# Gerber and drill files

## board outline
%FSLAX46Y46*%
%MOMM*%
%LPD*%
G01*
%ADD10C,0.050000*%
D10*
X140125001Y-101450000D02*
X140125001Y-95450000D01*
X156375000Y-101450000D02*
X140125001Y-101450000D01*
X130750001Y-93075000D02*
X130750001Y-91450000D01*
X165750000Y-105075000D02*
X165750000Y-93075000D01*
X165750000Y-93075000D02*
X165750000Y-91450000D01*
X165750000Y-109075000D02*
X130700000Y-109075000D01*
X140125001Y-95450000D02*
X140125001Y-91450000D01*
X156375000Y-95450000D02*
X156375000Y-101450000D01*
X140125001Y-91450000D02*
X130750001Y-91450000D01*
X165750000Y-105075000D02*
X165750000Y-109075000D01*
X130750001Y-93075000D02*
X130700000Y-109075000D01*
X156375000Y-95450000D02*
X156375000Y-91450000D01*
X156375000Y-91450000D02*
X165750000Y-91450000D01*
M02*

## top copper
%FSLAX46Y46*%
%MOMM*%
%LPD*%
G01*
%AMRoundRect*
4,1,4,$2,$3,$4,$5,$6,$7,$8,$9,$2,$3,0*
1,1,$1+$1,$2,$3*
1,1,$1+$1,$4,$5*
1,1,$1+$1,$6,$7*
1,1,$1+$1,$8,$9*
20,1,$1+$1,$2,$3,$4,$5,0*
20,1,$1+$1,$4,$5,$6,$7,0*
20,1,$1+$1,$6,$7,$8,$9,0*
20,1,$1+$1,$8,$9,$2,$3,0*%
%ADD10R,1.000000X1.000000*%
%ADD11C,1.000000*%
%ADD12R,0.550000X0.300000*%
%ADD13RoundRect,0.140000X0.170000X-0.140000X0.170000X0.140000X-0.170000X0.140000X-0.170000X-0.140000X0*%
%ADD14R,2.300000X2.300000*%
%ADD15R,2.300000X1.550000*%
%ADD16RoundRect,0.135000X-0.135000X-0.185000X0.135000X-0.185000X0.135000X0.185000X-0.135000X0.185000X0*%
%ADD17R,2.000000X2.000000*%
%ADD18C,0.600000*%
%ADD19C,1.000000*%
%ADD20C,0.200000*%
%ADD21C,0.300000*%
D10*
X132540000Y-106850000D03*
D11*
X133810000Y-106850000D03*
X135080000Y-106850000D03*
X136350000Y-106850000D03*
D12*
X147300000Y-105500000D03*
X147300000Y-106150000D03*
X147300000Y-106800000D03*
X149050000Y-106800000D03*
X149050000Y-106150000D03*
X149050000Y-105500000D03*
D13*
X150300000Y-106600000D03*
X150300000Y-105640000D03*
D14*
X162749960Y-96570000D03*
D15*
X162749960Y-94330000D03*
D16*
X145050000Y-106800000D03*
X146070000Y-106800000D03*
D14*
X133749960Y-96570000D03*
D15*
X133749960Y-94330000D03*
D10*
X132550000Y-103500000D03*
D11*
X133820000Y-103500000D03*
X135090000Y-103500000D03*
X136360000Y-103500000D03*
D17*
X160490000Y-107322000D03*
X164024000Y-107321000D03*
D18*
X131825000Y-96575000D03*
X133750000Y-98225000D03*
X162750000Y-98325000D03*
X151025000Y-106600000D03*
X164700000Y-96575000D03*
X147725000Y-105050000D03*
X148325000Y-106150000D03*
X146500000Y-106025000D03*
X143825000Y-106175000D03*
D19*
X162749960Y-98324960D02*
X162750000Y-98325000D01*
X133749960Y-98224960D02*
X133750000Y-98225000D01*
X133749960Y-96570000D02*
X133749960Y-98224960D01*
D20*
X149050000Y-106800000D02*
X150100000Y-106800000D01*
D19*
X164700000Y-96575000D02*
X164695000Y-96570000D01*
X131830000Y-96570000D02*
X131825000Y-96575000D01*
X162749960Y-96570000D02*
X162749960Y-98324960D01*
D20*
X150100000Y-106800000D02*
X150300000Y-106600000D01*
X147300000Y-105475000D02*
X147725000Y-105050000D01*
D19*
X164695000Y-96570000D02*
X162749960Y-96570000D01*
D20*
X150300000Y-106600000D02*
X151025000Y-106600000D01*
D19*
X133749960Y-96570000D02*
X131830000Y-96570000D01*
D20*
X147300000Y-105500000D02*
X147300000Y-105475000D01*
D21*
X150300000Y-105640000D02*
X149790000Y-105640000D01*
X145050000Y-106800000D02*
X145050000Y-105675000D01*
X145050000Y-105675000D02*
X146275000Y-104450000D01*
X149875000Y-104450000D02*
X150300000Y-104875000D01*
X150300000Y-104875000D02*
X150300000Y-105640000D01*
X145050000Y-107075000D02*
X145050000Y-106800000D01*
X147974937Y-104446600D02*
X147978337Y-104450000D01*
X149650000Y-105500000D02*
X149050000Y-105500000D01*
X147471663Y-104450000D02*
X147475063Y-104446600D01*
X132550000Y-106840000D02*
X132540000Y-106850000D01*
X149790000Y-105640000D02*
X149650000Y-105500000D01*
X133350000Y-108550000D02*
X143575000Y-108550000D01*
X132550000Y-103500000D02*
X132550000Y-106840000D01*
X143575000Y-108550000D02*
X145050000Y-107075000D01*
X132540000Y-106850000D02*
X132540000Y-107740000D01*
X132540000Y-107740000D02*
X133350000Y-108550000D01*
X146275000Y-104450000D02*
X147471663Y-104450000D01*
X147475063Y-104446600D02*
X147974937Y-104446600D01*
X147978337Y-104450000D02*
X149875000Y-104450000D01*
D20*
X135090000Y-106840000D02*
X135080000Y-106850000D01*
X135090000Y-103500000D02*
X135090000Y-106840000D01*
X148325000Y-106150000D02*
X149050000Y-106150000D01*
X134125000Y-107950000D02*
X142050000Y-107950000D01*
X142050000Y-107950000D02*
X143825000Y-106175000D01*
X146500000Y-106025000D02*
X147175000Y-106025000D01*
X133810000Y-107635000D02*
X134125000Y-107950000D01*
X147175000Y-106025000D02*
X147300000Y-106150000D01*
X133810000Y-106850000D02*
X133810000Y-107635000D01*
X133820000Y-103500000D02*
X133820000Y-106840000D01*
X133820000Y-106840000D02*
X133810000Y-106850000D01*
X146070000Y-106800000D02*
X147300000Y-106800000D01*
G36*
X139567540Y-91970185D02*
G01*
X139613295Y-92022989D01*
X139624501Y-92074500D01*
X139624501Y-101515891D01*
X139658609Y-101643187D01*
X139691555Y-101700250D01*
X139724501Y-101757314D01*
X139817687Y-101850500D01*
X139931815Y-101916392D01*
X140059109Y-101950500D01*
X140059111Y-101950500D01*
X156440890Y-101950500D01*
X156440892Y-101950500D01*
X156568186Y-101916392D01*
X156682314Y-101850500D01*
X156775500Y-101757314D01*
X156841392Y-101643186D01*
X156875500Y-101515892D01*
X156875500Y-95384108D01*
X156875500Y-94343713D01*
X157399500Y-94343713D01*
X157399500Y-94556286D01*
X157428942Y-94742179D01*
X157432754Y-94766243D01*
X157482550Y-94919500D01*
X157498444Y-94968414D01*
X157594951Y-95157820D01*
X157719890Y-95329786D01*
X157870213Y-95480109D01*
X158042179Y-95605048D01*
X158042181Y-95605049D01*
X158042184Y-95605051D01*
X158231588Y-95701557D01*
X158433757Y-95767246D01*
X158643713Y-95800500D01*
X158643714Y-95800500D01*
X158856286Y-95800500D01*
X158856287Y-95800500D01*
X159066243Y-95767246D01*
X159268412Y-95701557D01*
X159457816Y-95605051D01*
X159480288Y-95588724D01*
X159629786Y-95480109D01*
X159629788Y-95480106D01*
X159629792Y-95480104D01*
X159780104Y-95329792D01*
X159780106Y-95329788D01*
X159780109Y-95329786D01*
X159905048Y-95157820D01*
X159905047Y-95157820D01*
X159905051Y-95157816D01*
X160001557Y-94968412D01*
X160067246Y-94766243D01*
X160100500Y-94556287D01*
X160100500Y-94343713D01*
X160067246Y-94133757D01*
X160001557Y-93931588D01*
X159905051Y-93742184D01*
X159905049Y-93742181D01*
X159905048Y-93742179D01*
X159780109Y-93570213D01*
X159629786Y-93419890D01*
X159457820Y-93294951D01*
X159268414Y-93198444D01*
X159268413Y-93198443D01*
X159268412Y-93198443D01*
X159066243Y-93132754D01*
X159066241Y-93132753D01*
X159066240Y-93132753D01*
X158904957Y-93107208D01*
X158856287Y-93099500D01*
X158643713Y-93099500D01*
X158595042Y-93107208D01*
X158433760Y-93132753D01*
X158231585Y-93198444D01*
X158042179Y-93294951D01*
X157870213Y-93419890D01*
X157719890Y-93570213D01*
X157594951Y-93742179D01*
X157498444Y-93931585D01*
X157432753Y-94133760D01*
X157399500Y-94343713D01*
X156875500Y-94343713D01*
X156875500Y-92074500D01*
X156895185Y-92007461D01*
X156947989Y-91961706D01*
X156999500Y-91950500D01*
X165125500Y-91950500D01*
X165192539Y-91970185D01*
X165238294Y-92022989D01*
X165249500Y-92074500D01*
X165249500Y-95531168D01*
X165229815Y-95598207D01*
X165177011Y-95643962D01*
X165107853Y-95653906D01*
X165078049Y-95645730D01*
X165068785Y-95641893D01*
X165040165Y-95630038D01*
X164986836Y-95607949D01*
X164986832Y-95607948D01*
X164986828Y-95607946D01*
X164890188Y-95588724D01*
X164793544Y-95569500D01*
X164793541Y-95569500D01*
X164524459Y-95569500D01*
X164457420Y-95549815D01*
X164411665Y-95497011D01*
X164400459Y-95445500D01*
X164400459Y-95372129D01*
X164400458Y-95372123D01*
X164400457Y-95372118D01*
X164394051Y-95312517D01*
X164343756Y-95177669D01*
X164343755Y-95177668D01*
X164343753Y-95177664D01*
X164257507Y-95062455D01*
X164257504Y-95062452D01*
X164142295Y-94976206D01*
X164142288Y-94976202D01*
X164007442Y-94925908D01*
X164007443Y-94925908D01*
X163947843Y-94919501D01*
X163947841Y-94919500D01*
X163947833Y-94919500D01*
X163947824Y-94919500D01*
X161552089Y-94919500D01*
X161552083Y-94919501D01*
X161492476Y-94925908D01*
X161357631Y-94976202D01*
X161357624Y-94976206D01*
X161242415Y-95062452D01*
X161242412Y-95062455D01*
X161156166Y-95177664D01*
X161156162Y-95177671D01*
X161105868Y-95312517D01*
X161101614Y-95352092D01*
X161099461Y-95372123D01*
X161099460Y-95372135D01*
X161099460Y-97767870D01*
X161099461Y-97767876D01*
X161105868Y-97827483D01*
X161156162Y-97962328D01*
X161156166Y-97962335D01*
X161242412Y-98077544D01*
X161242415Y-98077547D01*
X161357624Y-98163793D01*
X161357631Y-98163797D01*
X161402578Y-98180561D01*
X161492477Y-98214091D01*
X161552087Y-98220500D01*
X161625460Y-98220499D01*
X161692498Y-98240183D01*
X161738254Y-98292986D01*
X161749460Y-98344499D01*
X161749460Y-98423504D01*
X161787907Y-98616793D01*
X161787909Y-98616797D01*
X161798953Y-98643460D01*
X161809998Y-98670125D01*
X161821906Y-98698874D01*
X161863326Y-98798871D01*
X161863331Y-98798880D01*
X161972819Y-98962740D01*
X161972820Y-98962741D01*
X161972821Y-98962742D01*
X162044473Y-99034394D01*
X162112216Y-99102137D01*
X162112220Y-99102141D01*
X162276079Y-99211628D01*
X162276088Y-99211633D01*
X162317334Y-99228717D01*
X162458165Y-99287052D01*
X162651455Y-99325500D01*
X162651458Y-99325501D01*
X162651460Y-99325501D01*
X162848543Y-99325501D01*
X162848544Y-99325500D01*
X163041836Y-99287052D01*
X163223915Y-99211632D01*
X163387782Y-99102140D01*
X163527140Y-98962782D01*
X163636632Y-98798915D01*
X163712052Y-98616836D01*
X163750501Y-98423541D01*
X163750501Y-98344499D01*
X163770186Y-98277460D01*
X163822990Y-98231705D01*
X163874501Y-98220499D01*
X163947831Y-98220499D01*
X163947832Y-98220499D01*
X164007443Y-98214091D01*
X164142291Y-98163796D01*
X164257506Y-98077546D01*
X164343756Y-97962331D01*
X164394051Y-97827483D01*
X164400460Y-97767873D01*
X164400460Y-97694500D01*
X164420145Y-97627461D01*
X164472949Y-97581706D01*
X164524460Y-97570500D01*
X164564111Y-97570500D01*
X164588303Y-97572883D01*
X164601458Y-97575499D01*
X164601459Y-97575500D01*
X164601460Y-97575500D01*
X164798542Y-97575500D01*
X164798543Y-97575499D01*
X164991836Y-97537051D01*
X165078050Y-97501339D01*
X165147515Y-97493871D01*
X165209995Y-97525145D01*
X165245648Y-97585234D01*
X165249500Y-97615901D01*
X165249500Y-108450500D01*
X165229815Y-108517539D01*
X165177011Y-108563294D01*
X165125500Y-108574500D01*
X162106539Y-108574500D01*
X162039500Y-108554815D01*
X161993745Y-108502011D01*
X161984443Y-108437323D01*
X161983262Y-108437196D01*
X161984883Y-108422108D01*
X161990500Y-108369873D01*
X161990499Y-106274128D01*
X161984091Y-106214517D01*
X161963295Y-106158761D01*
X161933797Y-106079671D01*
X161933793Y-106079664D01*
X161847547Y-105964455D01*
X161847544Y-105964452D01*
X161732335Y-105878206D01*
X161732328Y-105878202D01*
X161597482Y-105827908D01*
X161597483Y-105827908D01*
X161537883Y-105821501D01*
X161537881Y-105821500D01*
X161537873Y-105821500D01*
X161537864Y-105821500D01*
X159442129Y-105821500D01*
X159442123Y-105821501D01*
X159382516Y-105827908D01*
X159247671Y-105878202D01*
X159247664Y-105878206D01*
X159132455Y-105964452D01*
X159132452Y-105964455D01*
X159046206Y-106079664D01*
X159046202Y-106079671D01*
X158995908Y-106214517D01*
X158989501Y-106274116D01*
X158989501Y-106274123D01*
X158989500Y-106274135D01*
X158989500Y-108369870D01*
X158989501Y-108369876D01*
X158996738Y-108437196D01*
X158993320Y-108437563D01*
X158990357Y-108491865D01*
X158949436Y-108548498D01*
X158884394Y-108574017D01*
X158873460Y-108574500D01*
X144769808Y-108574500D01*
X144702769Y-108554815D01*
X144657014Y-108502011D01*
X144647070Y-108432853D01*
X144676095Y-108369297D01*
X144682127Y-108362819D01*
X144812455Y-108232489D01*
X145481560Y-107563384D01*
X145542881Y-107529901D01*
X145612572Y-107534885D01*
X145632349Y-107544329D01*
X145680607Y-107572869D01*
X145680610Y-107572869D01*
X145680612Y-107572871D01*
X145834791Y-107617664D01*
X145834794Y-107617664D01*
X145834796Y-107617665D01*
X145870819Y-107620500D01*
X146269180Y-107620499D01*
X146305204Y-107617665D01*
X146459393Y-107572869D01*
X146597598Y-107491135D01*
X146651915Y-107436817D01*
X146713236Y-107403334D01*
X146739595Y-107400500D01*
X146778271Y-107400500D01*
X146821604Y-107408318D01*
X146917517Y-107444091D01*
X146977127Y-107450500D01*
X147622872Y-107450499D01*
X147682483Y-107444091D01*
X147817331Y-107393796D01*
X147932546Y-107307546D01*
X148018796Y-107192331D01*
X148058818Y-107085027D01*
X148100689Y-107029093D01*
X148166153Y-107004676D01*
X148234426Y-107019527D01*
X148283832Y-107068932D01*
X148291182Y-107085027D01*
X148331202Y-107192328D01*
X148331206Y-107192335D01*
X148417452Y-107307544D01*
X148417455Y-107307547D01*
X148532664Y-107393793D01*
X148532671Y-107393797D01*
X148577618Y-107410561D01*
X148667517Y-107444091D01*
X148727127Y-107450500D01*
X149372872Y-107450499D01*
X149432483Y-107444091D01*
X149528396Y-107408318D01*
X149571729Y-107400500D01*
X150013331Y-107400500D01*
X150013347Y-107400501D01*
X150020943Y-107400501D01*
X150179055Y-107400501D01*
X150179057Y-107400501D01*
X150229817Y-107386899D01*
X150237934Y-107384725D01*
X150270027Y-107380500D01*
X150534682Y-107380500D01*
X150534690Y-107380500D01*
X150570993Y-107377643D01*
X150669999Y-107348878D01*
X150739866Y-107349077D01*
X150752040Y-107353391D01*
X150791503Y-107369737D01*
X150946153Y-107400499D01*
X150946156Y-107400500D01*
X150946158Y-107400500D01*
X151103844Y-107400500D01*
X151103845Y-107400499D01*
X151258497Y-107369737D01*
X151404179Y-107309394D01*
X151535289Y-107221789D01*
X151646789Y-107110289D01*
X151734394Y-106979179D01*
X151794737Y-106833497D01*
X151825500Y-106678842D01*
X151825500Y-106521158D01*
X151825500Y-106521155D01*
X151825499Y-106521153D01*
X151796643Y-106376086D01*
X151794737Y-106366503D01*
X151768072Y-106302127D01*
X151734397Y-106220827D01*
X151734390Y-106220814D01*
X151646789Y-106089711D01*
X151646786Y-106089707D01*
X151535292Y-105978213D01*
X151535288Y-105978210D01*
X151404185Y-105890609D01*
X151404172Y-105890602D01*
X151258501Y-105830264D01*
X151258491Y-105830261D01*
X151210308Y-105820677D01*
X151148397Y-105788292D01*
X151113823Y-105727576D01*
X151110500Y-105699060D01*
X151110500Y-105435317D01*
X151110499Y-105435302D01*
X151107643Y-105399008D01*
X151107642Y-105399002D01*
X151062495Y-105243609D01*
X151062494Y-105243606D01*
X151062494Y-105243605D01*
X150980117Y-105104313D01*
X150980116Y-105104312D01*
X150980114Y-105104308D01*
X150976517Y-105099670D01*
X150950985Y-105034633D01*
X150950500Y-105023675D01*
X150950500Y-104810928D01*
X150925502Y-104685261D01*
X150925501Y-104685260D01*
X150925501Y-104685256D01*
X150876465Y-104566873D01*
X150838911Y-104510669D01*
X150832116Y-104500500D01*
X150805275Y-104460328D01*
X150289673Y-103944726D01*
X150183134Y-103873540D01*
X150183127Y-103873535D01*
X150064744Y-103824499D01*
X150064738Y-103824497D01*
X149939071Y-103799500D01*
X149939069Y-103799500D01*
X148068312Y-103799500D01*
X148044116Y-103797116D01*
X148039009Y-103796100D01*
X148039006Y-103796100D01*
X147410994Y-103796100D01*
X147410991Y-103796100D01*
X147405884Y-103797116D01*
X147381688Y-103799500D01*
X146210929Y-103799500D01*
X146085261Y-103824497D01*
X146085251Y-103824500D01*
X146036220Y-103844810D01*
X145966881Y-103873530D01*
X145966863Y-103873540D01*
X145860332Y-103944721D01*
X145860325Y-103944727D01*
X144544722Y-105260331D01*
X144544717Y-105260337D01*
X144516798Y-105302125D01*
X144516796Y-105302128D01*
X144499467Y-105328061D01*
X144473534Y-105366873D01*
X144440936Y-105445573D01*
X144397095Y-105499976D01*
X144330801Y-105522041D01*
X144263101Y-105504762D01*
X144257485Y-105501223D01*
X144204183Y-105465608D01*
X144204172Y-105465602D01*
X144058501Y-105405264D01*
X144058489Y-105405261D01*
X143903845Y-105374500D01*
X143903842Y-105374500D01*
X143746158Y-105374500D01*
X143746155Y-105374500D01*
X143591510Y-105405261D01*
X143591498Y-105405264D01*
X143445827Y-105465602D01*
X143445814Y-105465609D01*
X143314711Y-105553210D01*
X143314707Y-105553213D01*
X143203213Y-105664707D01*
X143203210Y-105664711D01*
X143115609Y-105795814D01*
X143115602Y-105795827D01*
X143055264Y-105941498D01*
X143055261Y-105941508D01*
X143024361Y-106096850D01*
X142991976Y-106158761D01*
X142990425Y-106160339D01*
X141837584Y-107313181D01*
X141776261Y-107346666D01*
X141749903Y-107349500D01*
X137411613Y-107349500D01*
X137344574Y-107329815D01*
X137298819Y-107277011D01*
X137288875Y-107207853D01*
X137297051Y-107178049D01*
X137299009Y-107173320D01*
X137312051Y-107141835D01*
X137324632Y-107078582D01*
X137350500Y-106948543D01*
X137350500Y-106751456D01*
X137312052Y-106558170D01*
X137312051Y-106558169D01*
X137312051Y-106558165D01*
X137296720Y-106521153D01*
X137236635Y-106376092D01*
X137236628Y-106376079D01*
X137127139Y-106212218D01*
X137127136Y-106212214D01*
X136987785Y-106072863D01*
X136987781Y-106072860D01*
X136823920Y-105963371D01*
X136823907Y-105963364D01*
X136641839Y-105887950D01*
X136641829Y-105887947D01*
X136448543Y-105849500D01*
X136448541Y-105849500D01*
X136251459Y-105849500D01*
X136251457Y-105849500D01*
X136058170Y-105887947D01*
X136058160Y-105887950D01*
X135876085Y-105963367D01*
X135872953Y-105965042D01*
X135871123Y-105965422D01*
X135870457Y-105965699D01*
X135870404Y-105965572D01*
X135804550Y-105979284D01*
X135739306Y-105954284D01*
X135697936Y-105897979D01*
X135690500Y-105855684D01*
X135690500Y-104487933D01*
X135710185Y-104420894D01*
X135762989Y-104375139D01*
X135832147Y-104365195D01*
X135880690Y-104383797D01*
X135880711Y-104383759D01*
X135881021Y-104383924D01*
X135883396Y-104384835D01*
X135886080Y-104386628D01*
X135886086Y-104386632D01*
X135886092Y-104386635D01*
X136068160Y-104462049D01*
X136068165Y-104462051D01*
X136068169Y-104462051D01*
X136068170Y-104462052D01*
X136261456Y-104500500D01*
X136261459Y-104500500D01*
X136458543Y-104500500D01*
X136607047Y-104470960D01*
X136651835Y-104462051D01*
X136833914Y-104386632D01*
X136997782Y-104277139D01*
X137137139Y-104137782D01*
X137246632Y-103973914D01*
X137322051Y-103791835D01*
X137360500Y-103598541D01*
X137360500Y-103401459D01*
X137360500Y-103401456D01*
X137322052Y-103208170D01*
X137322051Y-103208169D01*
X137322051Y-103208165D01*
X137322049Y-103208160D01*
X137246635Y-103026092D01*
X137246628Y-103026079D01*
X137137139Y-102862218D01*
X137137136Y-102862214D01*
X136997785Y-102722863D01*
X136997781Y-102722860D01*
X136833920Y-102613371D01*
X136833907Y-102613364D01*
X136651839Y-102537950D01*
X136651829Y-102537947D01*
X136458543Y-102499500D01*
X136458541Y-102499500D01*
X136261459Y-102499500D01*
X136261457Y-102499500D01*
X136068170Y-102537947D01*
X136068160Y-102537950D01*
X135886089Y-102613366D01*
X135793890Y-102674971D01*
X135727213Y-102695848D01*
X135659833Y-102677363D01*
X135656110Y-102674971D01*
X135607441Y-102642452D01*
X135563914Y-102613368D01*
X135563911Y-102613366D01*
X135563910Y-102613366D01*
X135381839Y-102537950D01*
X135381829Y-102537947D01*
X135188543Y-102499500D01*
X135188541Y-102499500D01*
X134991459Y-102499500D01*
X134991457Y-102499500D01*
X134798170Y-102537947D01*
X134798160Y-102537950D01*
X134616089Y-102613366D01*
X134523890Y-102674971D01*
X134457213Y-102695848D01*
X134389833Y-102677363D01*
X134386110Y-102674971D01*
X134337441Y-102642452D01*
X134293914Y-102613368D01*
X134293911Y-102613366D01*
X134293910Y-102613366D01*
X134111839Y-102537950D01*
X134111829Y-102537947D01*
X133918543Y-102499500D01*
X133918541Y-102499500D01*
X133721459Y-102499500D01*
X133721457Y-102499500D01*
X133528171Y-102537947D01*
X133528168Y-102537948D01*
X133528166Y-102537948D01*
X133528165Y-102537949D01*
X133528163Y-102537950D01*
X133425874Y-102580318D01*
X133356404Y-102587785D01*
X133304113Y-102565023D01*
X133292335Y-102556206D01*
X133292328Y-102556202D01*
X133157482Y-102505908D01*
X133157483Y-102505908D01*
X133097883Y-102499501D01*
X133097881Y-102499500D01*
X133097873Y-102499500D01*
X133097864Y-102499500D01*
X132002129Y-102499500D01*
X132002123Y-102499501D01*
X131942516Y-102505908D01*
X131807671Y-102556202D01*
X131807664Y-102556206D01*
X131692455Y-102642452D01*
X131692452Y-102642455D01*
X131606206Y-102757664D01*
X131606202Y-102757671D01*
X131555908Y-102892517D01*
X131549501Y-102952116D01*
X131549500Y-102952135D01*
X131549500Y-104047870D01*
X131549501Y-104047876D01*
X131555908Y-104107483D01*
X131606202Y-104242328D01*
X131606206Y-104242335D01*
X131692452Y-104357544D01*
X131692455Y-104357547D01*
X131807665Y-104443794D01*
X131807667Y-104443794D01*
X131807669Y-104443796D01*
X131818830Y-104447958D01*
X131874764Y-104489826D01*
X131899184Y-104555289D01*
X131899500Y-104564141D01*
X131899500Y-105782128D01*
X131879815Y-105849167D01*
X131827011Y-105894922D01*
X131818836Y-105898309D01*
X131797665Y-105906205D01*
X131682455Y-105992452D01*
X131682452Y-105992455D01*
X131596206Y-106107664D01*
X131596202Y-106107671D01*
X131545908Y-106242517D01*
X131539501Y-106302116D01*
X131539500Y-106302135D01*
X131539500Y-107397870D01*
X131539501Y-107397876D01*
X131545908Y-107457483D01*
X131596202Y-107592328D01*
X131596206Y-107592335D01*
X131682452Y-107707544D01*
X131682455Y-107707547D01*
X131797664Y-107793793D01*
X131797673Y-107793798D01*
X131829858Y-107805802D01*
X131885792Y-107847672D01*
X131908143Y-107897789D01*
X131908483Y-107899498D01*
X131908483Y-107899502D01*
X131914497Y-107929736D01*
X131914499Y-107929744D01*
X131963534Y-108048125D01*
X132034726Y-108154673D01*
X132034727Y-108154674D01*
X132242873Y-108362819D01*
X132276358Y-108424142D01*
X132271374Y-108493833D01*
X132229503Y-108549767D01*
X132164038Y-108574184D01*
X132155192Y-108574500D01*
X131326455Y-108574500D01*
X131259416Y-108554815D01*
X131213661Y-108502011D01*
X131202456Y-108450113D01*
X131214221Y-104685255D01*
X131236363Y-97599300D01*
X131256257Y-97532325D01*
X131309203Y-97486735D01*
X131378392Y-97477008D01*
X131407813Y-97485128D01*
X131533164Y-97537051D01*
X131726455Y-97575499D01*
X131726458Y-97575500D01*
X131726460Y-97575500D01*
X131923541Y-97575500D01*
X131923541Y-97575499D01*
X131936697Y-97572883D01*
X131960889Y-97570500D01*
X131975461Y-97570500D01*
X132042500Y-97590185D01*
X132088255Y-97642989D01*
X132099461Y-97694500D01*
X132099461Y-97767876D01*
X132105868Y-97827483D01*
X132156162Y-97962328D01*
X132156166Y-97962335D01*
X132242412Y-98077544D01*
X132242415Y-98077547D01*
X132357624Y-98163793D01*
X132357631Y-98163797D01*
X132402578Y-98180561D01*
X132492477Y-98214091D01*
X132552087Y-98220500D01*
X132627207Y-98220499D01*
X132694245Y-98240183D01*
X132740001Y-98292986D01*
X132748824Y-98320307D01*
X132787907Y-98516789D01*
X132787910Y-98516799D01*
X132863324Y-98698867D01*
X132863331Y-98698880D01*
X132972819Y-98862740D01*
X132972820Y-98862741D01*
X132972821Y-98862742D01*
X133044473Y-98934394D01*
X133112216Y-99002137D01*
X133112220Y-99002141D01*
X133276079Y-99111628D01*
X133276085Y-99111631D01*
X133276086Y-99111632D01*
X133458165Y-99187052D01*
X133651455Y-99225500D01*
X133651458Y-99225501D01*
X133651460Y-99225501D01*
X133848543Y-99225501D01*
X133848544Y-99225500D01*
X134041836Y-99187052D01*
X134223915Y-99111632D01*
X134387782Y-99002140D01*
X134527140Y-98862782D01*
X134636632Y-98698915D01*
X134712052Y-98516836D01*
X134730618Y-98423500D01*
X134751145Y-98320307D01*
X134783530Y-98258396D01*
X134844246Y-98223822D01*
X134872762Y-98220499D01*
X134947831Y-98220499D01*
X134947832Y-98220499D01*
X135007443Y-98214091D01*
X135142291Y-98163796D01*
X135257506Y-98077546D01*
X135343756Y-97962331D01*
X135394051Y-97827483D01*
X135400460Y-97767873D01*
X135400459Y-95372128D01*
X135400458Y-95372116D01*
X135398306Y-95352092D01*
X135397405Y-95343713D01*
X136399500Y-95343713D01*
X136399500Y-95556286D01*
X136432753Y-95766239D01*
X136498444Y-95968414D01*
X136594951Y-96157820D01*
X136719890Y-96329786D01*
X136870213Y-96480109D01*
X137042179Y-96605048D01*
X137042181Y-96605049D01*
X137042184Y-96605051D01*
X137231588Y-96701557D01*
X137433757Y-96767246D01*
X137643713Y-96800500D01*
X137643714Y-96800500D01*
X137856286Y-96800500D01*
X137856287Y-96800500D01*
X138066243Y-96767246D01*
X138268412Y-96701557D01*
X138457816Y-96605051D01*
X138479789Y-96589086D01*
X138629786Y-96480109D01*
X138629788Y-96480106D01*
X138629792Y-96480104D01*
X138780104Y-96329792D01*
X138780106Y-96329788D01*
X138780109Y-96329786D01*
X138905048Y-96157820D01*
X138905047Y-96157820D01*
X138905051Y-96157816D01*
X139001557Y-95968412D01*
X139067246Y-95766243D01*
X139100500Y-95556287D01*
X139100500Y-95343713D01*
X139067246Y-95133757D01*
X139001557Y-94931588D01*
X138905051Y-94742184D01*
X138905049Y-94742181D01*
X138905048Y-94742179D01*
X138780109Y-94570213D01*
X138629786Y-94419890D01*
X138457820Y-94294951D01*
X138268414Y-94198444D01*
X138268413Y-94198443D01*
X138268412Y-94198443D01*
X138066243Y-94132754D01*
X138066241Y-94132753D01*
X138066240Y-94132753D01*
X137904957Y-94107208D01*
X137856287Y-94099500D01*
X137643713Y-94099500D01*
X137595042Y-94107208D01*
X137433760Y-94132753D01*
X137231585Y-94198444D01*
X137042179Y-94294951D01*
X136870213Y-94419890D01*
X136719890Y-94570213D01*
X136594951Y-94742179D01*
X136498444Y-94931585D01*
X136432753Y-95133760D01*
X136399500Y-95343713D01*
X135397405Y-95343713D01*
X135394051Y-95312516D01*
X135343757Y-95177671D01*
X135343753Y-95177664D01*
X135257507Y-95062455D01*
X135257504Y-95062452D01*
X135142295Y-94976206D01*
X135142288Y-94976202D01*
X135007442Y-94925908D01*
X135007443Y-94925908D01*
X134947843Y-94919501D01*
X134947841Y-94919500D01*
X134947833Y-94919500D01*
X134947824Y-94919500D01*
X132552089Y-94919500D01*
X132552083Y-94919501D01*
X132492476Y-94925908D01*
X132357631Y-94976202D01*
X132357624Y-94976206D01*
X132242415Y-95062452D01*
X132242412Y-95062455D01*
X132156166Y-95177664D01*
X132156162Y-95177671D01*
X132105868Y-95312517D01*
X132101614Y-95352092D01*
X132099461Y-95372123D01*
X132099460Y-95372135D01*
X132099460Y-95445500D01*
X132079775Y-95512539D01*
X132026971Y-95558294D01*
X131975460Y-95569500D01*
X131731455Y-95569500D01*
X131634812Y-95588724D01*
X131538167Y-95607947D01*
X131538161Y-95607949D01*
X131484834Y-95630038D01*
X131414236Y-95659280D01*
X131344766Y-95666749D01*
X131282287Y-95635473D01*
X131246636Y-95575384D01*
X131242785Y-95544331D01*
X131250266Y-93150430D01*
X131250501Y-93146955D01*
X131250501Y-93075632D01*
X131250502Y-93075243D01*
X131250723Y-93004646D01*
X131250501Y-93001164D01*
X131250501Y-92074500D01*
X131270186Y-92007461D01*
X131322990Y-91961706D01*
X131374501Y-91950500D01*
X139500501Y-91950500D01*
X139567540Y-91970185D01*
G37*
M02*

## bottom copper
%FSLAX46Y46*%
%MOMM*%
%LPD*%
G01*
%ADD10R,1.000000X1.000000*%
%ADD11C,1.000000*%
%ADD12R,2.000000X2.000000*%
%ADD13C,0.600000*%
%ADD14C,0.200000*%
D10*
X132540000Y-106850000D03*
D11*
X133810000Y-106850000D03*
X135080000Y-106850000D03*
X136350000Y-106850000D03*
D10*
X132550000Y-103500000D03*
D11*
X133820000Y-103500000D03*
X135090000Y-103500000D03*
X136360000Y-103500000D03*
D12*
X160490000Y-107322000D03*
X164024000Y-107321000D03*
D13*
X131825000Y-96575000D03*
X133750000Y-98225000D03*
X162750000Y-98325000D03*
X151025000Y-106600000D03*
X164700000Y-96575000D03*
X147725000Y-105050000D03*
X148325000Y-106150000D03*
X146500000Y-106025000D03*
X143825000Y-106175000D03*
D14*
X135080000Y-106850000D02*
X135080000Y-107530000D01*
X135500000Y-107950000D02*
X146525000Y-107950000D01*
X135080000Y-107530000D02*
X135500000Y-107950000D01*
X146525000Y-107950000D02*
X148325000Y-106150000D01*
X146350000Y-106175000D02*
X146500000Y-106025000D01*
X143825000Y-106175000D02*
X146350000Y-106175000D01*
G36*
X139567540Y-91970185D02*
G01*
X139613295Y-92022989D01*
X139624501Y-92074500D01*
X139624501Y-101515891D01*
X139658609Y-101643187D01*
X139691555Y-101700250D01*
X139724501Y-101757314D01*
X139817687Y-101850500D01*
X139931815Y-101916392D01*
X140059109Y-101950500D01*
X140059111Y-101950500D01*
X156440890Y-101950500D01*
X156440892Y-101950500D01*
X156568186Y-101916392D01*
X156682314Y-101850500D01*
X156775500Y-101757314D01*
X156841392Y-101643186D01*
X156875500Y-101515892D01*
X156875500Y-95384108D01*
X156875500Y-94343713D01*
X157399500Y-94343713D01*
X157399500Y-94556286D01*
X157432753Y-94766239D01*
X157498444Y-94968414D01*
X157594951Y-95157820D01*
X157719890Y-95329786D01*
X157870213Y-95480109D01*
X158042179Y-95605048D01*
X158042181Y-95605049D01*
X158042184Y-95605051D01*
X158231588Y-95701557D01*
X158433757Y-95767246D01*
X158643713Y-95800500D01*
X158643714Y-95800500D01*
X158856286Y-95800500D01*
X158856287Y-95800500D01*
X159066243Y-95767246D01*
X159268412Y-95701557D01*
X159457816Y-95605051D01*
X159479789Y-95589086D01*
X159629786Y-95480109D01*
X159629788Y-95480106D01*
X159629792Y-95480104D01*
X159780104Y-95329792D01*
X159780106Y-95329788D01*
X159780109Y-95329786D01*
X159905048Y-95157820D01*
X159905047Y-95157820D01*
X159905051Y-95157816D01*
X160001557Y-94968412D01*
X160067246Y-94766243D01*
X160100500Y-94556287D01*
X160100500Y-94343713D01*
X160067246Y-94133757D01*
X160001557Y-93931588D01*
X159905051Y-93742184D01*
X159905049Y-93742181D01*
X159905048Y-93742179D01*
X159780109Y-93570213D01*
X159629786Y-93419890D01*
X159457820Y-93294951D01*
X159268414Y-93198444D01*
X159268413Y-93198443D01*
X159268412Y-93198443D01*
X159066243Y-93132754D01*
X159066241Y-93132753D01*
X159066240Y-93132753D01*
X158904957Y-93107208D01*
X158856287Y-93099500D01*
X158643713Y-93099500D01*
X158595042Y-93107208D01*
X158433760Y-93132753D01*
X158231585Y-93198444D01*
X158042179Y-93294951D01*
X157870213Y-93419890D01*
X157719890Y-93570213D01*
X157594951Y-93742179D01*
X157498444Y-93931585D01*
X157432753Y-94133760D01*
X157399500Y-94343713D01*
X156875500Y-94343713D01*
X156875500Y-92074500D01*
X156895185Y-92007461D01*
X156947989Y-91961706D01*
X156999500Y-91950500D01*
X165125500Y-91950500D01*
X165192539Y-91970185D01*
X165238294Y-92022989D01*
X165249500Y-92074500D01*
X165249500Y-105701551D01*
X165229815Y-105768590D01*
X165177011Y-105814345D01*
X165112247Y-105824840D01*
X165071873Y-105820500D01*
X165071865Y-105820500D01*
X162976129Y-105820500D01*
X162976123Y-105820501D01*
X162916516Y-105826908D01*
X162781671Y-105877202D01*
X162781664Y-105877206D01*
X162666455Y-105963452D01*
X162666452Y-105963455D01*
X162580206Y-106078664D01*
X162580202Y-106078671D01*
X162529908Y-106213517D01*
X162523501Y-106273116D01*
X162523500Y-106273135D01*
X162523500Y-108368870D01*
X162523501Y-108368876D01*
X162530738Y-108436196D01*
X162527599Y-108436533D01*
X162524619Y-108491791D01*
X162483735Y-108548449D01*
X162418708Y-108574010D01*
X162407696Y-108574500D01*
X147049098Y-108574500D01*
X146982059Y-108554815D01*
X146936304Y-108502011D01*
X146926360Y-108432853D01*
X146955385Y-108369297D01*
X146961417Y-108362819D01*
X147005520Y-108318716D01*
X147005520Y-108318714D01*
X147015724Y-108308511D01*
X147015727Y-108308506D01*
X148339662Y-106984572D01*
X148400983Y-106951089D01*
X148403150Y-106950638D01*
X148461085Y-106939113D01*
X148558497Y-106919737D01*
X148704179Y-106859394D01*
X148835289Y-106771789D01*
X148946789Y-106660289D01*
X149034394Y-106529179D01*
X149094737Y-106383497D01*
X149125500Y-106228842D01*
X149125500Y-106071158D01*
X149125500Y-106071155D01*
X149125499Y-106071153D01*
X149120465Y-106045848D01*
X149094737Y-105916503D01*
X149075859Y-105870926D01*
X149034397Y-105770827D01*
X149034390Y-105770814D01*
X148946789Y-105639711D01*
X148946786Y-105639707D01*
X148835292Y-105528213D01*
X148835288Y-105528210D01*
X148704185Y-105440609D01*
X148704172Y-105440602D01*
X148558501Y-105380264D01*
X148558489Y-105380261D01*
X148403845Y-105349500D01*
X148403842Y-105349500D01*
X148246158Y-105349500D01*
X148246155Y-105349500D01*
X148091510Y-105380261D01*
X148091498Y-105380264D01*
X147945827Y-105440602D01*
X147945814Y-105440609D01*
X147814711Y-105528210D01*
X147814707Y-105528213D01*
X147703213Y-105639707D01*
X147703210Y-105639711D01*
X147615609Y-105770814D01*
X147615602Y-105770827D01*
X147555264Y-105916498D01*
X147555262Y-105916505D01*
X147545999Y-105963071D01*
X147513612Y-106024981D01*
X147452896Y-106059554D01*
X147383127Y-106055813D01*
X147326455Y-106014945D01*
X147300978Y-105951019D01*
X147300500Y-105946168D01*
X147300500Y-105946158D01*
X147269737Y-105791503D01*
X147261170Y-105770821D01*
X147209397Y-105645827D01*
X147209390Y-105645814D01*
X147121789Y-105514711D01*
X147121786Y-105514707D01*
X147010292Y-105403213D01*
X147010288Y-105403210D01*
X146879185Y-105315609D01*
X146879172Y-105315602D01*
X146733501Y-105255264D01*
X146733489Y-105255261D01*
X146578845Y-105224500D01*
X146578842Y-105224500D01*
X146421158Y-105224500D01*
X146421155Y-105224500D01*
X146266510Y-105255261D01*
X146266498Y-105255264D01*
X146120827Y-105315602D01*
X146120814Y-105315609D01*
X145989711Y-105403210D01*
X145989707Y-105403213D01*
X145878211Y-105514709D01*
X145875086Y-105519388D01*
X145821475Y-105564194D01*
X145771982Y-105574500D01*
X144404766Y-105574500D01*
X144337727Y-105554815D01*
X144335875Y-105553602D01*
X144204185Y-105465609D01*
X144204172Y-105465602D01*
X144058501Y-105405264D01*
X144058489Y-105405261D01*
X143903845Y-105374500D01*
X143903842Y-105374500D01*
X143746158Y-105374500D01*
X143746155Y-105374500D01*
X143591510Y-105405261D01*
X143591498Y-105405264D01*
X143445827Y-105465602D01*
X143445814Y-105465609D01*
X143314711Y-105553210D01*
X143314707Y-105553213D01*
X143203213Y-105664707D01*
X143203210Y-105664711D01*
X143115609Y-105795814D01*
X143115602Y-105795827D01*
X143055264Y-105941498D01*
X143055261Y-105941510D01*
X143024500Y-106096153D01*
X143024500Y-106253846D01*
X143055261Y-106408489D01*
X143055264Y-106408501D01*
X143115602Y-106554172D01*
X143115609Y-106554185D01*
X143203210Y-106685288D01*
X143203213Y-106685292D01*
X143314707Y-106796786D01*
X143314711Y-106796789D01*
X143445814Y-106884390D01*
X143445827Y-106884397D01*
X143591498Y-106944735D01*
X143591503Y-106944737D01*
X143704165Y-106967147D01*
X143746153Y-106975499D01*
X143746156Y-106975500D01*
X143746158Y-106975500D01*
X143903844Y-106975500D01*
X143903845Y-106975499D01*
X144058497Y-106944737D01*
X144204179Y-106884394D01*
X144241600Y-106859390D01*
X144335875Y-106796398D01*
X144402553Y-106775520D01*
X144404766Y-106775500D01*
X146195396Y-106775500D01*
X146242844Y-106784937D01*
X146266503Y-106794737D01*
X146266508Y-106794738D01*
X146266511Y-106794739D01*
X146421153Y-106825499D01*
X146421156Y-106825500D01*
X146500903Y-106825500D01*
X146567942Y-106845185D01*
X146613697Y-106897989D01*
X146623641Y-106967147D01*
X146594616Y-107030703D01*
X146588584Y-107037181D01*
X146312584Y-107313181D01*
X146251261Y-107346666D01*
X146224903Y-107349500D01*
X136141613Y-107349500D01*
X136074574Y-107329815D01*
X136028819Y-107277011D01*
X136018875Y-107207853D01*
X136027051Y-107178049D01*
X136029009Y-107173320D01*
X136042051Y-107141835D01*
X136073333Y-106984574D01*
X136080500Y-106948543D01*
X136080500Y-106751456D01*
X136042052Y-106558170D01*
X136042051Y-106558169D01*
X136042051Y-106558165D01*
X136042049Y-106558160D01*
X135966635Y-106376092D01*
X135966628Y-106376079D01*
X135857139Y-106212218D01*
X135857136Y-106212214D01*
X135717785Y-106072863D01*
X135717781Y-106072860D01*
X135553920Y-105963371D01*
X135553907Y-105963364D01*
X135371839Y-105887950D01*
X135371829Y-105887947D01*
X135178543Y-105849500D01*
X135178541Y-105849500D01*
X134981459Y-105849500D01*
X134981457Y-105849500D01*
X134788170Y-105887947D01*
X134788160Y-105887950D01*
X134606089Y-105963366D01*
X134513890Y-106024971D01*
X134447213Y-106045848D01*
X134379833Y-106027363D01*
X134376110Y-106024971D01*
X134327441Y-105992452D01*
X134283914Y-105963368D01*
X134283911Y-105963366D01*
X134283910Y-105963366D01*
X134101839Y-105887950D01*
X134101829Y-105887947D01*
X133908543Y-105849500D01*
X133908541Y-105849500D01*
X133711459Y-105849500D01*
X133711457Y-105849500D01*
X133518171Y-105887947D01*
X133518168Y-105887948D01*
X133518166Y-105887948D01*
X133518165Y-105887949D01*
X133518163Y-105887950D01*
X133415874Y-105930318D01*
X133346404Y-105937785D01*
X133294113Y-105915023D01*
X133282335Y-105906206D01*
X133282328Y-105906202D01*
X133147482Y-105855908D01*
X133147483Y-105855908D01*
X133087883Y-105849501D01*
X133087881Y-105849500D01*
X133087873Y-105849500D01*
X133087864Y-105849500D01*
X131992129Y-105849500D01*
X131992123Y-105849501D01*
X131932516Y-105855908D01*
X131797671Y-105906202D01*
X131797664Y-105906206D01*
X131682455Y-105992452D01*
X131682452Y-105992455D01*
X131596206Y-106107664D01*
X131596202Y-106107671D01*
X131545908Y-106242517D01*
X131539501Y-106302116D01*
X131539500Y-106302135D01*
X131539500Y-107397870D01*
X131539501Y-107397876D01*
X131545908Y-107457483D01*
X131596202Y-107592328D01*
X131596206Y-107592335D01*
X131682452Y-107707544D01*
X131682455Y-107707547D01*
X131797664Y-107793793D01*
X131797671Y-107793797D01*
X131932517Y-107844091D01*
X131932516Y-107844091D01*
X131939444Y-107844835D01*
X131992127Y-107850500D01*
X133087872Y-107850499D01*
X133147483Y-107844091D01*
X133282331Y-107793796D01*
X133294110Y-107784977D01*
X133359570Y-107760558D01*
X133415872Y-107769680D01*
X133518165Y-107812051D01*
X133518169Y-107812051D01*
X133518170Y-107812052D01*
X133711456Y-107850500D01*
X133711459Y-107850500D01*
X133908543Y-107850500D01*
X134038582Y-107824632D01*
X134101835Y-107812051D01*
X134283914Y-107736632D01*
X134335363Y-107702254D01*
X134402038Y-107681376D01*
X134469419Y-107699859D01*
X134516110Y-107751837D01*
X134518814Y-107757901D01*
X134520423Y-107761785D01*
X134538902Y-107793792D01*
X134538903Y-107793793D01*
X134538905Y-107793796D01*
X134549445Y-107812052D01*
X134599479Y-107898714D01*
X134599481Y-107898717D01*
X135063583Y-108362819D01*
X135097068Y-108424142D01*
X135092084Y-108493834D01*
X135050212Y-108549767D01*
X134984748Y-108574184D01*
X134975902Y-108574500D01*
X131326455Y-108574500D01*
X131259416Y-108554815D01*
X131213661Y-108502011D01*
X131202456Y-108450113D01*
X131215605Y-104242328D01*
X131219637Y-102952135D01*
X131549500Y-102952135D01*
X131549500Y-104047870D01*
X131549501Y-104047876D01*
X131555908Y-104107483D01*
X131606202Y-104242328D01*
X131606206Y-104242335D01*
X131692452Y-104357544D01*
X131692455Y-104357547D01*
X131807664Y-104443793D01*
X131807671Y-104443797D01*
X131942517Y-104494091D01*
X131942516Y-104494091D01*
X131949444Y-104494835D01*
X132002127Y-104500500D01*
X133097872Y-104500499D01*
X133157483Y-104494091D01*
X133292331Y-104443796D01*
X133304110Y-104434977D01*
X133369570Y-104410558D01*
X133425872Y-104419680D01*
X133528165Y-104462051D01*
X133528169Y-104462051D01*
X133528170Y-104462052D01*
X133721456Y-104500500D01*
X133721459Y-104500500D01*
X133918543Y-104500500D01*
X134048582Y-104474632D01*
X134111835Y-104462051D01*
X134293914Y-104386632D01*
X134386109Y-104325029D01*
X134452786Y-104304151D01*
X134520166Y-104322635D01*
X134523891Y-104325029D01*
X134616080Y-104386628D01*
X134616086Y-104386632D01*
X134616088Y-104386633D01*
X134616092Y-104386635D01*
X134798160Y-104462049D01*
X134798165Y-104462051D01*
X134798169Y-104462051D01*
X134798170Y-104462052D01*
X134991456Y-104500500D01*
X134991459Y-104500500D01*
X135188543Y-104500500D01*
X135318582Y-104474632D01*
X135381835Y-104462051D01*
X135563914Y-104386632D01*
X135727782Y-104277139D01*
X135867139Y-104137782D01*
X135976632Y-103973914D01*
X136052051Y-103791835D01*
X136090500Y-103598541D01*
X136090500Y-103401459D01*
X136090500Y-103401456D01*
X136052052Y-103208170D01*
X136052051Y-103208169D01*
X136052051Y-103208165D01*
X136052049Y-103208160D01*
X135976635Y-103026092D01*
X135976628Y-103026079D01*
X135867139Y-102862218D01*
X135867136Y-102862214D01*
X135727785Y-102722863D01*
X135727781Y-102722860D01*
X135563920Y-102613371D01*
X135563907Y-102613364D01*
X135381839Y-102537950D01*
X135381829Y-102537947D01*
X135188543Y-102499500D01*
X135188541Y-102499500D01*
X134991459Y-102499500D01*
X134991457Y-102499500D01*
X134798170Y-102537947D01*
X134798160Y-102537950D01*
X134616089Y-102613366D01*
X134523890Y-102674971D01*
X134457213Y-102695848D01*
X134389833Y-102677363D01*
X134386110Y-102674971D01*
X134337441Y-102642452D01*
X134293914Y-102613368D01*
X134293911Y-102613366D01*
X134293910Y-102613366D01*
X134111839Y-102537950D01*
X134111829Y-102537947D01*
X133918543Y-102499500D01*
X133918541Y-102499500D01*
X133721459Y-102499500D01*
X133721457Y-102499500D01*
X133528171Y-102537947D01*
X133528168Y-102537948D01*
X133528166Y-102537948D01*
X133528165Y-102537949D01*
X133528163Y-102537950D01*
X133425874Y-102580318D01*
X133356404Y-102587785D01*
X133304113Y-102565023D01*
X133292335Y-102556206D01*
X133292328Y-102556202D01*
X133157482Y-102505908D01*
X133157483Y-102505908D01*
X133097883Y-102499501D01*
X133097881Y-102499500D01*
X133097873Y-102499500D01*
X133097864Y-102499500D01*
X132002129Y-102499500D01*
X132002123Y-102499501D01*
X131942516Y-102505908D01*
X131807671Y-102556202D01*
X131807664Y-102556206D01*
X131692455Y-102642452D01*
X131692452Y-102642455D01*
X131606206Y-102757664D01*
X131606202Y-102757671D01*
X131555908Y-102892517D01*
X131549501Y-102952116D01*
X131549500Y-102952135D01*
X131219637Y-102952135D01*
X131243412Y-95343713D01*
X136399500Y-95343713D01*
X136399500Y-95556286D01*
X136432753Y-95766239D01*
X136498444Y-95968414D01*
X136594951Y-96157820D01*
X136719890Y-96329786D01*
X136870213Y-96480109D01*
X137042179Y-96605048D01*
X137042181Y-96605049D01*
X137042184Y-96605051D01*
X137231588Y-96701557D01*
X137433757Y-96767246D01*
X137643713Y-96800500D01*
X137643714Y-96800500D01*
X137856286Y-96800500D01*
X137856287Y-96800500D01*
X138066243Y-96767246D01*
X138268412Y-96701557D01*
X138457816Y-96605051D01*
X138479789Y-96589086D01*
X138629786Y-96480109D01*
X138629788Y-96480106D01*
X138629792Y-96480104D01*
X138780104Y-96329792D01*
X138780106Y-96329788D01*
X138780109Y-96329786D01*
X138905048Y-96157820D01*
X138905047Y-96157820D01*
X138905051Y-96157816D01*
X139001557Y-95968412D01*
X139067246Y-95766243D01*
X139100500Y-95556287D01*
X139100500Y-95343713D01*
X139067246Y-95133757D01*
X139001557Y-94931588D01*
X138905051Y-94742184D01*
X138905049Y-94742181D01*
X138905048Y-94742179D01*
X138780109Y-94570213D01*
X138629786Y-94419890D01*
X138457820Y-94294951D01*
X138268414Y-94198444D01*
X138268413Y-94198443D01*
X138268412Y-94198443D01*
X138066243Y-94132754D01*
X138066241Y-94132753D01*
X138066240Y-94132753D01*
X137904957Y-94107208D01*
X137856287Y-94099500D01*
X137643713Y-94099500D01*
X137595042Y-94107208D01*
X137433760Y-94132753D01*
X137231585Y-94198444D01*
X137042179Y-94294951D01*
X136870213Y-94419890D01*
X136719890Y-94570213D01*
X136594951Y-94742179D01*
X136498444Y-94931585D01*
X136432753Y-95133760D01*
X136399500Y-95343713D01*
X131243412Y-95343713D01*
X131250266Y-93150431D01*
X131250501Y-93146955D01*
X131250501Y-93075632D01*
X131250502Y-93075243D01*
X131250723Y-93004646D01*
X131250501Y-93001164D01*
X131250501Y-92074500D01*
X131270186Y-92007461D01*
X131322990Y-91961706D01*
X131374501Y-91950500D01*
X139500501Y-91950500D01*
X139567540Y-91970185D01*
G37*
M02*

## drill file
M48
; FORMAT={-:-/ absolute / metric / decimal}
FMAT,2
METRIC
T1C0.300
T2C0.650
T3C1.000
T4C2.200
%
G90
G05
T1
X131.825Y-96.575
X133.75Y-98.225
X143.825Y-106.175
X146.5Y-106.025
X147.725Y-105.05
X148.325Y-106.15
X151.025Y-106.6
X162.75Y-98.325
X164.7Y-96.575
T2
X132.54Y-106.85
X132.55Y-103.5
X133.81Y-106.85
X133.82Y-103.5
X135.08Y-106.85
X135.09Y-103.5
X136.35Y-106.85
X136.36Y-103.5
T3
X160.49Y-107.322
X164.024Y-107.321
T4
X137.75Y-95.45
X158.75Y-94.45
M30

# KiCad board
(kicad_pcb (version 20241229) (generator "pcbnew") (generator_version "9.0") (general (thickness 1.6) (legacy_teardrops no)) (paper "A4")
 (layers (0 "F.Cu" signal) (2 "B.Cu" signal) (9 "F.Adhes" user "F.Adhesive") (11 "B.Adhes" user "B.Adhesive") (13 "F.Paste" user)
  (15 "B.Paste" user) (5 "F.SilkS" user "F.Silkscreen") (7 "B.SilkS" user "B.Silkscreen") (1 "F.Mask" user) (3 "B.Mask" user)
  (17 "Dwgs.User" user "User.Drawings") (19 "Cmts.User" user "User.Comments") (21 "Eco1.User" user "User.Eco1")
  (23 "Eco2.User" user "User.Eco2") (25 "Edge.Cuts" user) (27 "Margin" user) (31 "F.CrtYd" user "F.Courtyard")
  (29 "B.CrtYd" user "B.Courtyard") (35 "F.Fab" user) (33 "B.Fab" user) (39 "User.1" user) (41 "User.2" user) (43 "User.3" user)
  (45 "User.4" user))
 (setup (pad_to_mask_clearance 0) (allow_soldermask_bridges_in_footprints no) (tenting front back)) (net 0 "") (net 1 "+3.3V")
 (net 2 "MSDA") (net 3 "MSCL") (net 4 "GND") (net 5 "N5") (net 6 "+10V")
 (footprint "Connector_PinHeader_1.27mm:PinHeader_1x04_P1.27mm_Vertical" (layer "F.Cu") (at 132.54 106.85 90)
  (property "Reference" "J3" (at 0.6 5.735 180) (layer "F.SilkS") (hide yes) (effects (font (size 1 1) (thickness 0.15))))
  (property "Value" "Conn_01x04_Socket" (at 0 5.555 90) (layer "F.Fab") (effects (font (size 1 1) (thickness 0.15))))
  (pad "1" thru_hole rect (at 0 0 90) (size 1 1) (drill 0.65) (layers "*.Cu" "*.Mask") (remove_unused_layers no) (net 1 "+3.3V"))
  (pad "2" thru_hole circle (at 0 1.27 90) (size 1 1) (drill 0.65) (layers "*.Cu" "*.Mask") (remove_unused_layers no) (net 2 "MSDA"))
  (pad "3" thru_hole circle (at 0 2.54 90) (size 1 1) (drill 0.65) (layers "*.Cu" "*.Mask") (remove_unused_layers no) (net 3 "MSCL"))
  (pad "4" thru_hole circle (at 0 3.81 90) (size 1 1) (drill 0.65) (layers "*.Cu" "*.Mask") (remove_unused_layers no) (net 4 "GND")))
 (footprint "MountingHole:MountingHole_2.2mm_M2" (layer "F.Cu") (at 137.75 95.45)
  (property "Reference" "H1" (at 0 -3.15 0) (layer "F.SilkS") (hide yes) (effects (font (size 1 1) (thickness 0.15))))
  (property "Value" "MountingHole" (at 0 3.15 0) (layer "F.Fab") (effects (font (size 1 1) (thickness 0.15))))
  (pad "" np_thru_hole circle (at 0 0) (size 2.2 2.2) (drill 2.2) (layers "*.Cu" "*.Mask")))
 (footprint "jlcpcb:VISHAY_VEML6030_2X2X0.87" (layer "F.Cu") (at 148.175 106.15)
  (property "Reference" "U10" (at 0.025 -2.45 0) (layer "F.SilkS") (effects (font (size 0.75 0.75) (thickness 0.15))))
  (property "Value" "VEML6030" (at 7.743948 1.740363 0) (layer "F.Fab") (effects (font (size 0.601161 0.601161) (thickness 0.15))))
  (pad "1" smd rect (at -0.875 -0.65) (size 0.55 0.3) (layers "F.Cu" "F.Mask" "F.Paste") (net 4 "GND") (solder_mask_margin 0.102))
  (pad "2" smd rect (at -0.875 0) (size 0.55 0.3) (layers "F.Cu" "F.Mask" "F.Paste") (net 2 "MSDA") (solder_mask_margin 0.102))
  (pad "3" smd rect (at -0.875 0.65) (size 0.55 0.3) (layers "F.Cu" "F.Mask" "F.Paste") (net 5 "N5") (solder_mask_margin 0.102))
  (pad "4" smd rect (at 0.875 0.65) (size 0.55 0.3) (layers "F.Cu" "F.Mask" "F.Paste") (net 4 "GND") (solder_mask_margin 0.102))
  (pad "5" smd rect (at 0.875 0) (size 0.55 0.3) (layers "F.Cu" "F.Mask" "F.Paste") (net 3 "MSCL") (solder_mask_margin 0.102))
  (pad "6" smd rect (at 0.875 -0.65) (size 0.55 0.3) (layers "F.Cu" "F.Mask" "F.Paste") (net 1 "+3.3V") (solder_mask_margin 0.102)))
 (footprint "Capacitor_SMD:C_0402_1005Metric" (layer "F.Cu") (at 150.3 106.12 90)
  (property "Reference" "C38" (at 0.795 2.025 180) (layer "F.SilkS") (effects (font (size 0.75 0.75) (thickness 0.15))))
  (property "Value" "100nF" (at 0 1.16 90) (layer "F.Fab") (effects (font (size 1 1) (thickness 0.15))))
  (pad "1" smd roundrect (at -0.48 0 90) (size 0.56 0.62) (layers "F.Cu" "F.Mask" "F.Paste") (roundrect_rratio 0.25) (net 4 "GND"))
  (pad "2" smd roundrect (at 0.48 0 90) (size 0.56 0.62) (layers "F.Cu" "F.Mask" "F.Paste") (roundrect_rratio 0.25) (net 1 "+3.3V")))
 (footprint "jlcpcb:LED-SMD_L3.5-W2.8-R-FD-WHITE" (layer "F.Cu") (at 162.74996 95.45 -90)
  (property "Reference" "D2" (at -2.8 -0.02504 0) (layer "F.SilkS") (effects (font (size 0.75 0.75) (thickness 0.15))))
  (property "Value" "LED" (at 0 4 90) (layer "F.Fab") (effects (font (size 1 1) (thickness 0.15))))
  (pad "1" smd rect (at 1.12 0 270) (size 2.3 2.3) (layers "F.Cu" "F.Mask" "F.Paste") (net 4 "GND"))
  (pad "2" smd rect (at -1.12 0 270) (size 1.55 2.3) (layers "F.Cu" "F.Mask" "F.Paste") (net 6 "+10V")))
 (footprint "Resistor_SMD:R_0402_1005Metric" (layer "F.Cu") (at 145.56 106.8)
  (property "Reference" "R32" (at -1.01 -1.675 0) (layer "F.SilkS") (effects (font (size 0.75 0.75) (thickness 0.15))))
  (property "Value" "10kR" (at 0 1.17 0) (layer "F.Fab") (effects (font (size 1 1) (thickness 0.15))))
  (pad "1" smd roundrect (at -0.51 0) (size 0.54 0.64) (layers "F.Cu" "F.Mask" "F.Paste") (roundrect_rratio 0.25) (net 1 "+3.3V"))
  (pad "2" smd roundrect (at 0.51 0) (size 0.54 0.64) (layers "F.Cu" "F.Mask" "F.Paste") (roundrect_rratio 0.25) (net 5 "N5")))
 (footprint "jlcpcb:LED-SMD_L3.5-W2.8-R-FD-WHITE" (layer "F.Cu") (at 133.74996 95.45 -90)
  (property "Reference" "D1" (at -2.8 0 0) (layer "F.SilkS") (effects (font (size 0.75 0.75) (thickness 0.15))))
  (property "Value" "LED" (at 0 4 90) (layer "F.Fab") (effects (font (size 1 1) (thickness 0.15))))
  (pad "1" smd rect (at 1.12 0 270) (size 2.3 2.3) (layers "F.Cu" "F.Mask" "F.Paste") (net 4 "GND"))
  (pad "2" smd rect (at -1.12 0 270) (size 1.55 2.3) (layers "F.Cu" "F.Mask" "F.Paste") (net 6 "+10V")))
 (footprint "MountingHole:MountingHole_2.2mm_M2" (layer "F.Cu") (at 158.75 94.45)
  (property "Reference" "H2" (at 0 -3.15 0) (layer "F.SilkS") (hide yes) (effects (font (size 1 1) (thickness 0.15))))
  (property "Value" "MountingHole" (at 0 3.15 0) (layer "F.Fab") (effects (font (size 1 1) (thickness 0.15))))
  (pad "" np_thru_hole circle (at 0 0) (size 2.2 2.2) (drill 2.2) (layers "*.Cu" "*.Mask")))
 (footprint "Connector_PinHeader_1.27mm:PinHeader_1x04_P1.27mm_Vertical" (layer "F.Cu") (at 132.55 103.5 90)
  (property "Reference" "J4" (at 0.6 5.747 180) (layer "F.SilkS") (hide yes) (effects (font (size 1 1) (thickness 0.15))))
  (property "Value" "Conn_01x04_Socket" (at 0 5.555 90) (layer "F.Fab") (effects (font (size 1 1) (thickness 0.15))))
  (pad "1" thru_hole rect (at 0 0 90) (size 1 1) (drill 0.65) (layers "*.Cu" "*.Mask") (remove_unused_layers no) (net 1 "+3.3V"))
  (pad "2" thru_hole circle (at 0 1.27 90) (size 1 1) (drill 0.65) (layers "*.Cu" "*.Mask") (remove_unused_layers no) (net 2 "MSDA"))
  (pad "3" thru_hole circle (at 0 2.54 90) (size 1 1) (drill 0.65) (layers "*.Cu" "*.Mask") (remove_unused_layers no) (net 3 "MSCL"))
  (pad "4" thru_hole circle (at 0 3.81 90) (size 1 1) (drill 0.65) (layers "*.Cu" "*.Mask") (remove_unused_layers no) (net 4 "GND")))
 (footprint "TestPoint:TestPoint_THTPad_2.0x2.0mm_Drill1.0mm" (layer "B.Cu") (at 160.49 107.322)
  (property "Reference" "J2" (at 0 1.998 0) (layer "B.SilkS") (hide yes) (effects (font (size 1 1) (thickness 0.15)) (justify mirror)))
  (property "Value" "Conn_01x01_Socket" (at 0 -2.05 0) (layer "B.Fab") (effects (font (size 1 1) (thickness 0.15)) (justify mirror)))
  (pad "1" thru_hole rect (at 0 0) (size 2 2) (drill 1) (layers "*.Cu" "*.Mask") (remove_unused_layers no) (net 4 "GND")))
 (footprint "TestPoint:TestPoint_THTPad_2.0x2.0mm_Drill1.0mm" (layer "B.Cu") (at 164.024 107.321)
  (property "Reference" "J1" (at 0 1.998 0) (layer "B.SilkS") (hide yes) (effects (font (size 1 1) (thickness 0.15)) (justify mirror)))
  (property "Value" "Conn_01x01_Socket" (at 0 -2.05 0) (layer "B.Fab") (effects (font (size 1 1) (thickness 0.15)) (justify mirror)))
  (pad "1" thru_hole rect (at 0 0) (size 2 2) (drill 1) (layers "*.Cu" "*.Mask") (remove_unused_layers no) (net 6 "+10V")))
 (gr_line (start 140.125001 101.45) (end 140.125001 95.45) (stroke (width 0.05) (type solid)) (layer "Edge.Cuts"))
 (gr_line (start 156.375 101.45) (end 140.125001 101.45) (stroke (width 0.05) (type solid)) (layer "Edge.Cuts"))
 (gr_line (start 130.750001 93.075) (end 130.750001 91.45) (stroke (width 0.05) (type solid)) (layer "Edge.Cuts"))
 (gr_line (start 165.75 105.075) (end 165.75 93.075) (stroke (width 0.05) (type solid)) (layer "Edge.Cuts"))
 (gr_line (start 165.75 93.075) (end 165.75 91.45) (stroke (width 0.05) (type solid)) (layer "Edge.Cuts"))
 (gr_line (start 165.75 109.075) (end 130.7 109.075) (stroke (width 0.05) (type solid)) (layer "Edge.Cuts"))
 (gr_line (start 140.125001 95.45) (end 140.125001 91.45) (stroke (width 0.05) (type default)) (layer "Edge.Cuts"))
 (gr_line (start 156.375 95.45) (end 156.375 101.45) (stroke (width 0.05) (type solid)) (layer "Edge.Cuts"))
 (gr_line (start 140.125001 91.45) (end 130.750001 91.45) (stroke (width 0.05) (type solid)) (layer "Edge.Cuts"))
 (gr_line (start 165.75 105.075) (end 165.75 109.075) (stroke (width 0.05) (type solid)) (layer "Edge.Cuts"))
 (gr_line (start 130.750001 93.075) (end 130.7 109.075) (stroke (width 0.05) (type solid)) (layer "Edge.Cuts"))
 (gr_line (start 156.375 95.45) (end 156.375 91.45) (stroke (width 0.05) (type default)) (layer "Edge.Cuts"))
 (gr_line (start 156.375 91.45) (end 165.75 91.45) (stroke (width 0.05) (type solid)) (layer "Edge.Cuts"))
 (segment (start 162.74996 98.32496) (end 162.75 98.325) (width 1) (layer "F.Cu") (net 4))
 (segment (start 133.74996 98.22496) (end 133.75 98.225) (width 1) (layer "F.Cu") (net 4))
 (segment (start 133.74996 96.57) (end 133.74996 98.22496) (width 1) (layer "F.Cu") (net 4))
 (segment (start 149.05 106.8) (end 150.1 106.8) (width 0.2) (layer "F.Cu") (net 4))
 (segment (start 164.7 96.575) (end 164.695 96.57) (width 1) (layer "F.Cu") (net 4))
 (segment (start 131.83 96.57) (end 131.825 96.575) (width 1) (layer "F.Cu") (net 4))
 (segment (start 162.74996 96.57) (end 162.74996 98.32496) (width 1) (layer "F.Cu") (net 4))
 (segment (start 150.1 106.8) (end 150.3 106.6) (width 0.2) (layer "F.Cu") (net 4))
 (segment (start 147.3 105.475) (end 147.725 105.05) (width 0.2) (layer "F.Cu") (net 4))
 (segment (start 164.695 96.57) (end 162.74996 96.57) (width 1) (layer "F.Cu") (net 4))
 (segment (start 150.3 106.6) (end 151.025 106.6) (width 0.2) (layer "F.Cu") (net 4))
 (segment (start 133.74996 96.57) (end 131.83 96.57) (width 1) (layer "F.Cu") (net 4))
 (segment (start 147.3 105.5) (end 147.3 105.475) (width 0.2) (layer "F.Cu") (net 4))
 (via (at 131.825 96.575) (size 0.6) (drill 0.3) (layers "F.Cu" "B.Cu") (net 4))
 (via (at 133.75 98.225) (size 0.6) (drill 0.3) (layers "F.Cu" "B.Cu") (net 4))
 (via (at 162.75 98.325) (size 0.6) (drill 0.3) (layers "F.Cu" "B.Cu") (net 4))
 (via (at 151.025 106.6) (size 0.6) (drill 0.3) (layers "F.Cu" "B.Cu") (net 4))
 (via (at 164.7 96.575) (size 0.6) (drill 0.3) (layers "F.Cu" "B.Cu") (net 4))
 (via (at 147.725 105.05) (size 0.6) (drill 0.3) (layers "F.Cu" "B.Cu") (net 4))
 (segment (start 150.3 105.64) (end 149.79 105.64) (width 0.3) (layer "F.Cu") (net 1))
 (segment (start 145.05 106.8) (end 145.05 105.675) (width 0.3) (layer "F.Cu") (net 1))
 (segment (start 145.05 105.675) (end 146.275 104.45) (width 0.3) (layer "F.Cu") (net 1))
 (segment (start 149.875 104.45) (end 150.3 104.875) (width 0.3) (layer "F.Cu") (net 1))
 (segment (start 150.3 104.875) (end 150.3 105.64) (width 0.3) (layer "F.Cu") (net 1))
 (segment (start 145.05 107.075) (end 145.05 106.8) (width 0.3) (layer "F.Cu") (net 1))
 (segment (start 147.974937 104.4466) (end 147.978337 104.45) (width 0.3) (layer "F.Cu") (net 1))
 (segment (start 149.65 105.5) (end 149.05 105.5) (width 0.3) (layer "F.Cu") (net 1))
 (segment (start 147.471663 104.45) (end 147.475063 104.4466) (width 0.3) (layer "F.Cu") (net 1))
 (segment (start 132.55 106.84) (end 132.54 106.85) (width 0.3) (layer "F.Cu") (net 1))
 (segment (start 149.79 105.64) (end 149.65 105.5) (width 0.3) (layer "F.Cu") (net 1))
 (segment (start 133.35 108.55) (end 143.575 108.55) (width 0.3) (layer "F.Cu") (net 1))
 (segment (start 132.55 103.5) (end 132.55 106.84) (width 0.3) (layer "F.Cu") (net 1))
 (segment (start 143.575 108.55) (end 145.05 107.075) (width 0.3) (layer "F.Cu") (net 1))
 (segment (start 132.54 106.85) (end 132.54 107.74) (width 0.3) (layer "F.Cu") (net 1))
 (segment (start 132.54 107.74) (end 133.35 108.55) (width 0.3) (layer "F.Cu") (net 1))
 (segment (start 146.275 104.45) (end 147.471663 104.45) (width 0.3) (layer "F.Cu") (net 1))
 (segment (start 147.475063 104.4466) (end 147.974937 104.4466) (width 0.3) (layer "F.Cu") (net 1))
 (segment (start 147.978337 104.45) (end 149.875 104.45) (width 0.3) (layer "F.Cu") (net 1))
 (segment (start 135.09 106.84) (end 135.08 106.85) (width 0.2) (layer "F.Cu") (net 3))
 (segment (start 135.09 103.5) (end 135.09 106.84) (width 0.2) (layer "F.Cu") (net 3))
 (segment (start 148.325 106.15) (end 149.05 106.15) (width 0.2) (layer "F.Cu") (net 3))
 (via (at 148.325 106.15) (size 0.6) (drill 0.3) (layers "F.Cu" "B.Cu") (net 3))
 (segment (start 135.08 106.85) (end 135.08 107.53) (width 0.2) (layer "B.Cu") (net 3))
 (segment (start 135.5 107.95) (end 146.525 107.95) (width 0.2) (layer "B.Cu") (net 3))
 (segment (start 135.08 107.53) (end 135.5 107.95) (width 0.2) (layer "B.Cu") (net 3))
 (segment (start 146.525 107.95) (end 148.325 106.15) (width 0.2) (layer "B.Cu") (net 3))
 (segment (start 134.125 107.95) (end 142.05 107.95) (width 0.2) (layer "F.Cu") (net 2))
 (segment (start 142.05 107.95) (end 143.825 106.175) (width 0.2) (layer "F.Cu") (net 2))
 (segment (start 146.5 106.025) (end 147.175 106.025) (width 0.2) (layer "F.Cu") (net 2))
 (segment (start 133.81 107.635) (end 134.125 107.95) (width 0.2) (layer "F.Cu") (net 2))
 (segment (start 147.175 106.025) (end 147.3 106.15) (width 0.2) (layer "F.Cu") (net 2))
 (segment (start 133.81 106.85) (end 133.81 107.635) (width 0.2) (layer "F.Cu") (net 2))
 (segment (start 133.82 103.5) (end 133.82 106.84) (width 0.2) (layer "F.Cu") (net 2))
 (segment (start 133.82 106.84) (end 133.81 106.85) (width 0.2) (layer "F.Cu") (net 2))
 (via (at 146.5 106.025) (size 0.6) (drill 0.3) (layers "F.Cu" "B.Cu") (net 2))
 (via (at 143.825 106.175) (size 0.6) (drill 0.3) (layers "F.Cu" "B.Cu") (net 2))
 (segment (start 146.35 106.175) (end 146.5 106.025) (width 0.2) (layer "B.Cu") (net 2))
 (segment (start 143.825 106.175) (end 146.35 106.175) (width 0.2) (layer "B.Cu") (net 2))
 (segment (start 146.07 106.8) (end 147.3 106.8) (width 0.2) (layer "F.Cu") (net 5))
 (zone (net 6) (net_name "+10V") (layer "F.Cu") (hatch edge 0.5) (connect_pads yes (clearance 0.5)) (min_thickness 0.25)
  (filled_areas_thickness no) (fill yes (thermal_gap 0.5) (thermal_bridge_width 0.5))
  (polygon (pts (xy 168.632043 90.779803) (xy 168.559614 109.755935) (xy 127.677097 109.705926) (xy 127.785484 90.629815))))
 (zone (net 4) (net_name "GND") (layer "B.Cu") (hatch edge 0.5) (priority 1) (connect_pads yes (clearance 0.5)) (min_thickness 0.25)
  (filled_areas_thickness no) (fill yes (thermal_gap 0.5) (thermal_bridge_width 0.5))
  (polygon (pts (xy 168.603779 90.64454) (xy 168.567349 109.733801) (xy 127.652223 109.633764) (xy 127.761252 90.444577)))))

